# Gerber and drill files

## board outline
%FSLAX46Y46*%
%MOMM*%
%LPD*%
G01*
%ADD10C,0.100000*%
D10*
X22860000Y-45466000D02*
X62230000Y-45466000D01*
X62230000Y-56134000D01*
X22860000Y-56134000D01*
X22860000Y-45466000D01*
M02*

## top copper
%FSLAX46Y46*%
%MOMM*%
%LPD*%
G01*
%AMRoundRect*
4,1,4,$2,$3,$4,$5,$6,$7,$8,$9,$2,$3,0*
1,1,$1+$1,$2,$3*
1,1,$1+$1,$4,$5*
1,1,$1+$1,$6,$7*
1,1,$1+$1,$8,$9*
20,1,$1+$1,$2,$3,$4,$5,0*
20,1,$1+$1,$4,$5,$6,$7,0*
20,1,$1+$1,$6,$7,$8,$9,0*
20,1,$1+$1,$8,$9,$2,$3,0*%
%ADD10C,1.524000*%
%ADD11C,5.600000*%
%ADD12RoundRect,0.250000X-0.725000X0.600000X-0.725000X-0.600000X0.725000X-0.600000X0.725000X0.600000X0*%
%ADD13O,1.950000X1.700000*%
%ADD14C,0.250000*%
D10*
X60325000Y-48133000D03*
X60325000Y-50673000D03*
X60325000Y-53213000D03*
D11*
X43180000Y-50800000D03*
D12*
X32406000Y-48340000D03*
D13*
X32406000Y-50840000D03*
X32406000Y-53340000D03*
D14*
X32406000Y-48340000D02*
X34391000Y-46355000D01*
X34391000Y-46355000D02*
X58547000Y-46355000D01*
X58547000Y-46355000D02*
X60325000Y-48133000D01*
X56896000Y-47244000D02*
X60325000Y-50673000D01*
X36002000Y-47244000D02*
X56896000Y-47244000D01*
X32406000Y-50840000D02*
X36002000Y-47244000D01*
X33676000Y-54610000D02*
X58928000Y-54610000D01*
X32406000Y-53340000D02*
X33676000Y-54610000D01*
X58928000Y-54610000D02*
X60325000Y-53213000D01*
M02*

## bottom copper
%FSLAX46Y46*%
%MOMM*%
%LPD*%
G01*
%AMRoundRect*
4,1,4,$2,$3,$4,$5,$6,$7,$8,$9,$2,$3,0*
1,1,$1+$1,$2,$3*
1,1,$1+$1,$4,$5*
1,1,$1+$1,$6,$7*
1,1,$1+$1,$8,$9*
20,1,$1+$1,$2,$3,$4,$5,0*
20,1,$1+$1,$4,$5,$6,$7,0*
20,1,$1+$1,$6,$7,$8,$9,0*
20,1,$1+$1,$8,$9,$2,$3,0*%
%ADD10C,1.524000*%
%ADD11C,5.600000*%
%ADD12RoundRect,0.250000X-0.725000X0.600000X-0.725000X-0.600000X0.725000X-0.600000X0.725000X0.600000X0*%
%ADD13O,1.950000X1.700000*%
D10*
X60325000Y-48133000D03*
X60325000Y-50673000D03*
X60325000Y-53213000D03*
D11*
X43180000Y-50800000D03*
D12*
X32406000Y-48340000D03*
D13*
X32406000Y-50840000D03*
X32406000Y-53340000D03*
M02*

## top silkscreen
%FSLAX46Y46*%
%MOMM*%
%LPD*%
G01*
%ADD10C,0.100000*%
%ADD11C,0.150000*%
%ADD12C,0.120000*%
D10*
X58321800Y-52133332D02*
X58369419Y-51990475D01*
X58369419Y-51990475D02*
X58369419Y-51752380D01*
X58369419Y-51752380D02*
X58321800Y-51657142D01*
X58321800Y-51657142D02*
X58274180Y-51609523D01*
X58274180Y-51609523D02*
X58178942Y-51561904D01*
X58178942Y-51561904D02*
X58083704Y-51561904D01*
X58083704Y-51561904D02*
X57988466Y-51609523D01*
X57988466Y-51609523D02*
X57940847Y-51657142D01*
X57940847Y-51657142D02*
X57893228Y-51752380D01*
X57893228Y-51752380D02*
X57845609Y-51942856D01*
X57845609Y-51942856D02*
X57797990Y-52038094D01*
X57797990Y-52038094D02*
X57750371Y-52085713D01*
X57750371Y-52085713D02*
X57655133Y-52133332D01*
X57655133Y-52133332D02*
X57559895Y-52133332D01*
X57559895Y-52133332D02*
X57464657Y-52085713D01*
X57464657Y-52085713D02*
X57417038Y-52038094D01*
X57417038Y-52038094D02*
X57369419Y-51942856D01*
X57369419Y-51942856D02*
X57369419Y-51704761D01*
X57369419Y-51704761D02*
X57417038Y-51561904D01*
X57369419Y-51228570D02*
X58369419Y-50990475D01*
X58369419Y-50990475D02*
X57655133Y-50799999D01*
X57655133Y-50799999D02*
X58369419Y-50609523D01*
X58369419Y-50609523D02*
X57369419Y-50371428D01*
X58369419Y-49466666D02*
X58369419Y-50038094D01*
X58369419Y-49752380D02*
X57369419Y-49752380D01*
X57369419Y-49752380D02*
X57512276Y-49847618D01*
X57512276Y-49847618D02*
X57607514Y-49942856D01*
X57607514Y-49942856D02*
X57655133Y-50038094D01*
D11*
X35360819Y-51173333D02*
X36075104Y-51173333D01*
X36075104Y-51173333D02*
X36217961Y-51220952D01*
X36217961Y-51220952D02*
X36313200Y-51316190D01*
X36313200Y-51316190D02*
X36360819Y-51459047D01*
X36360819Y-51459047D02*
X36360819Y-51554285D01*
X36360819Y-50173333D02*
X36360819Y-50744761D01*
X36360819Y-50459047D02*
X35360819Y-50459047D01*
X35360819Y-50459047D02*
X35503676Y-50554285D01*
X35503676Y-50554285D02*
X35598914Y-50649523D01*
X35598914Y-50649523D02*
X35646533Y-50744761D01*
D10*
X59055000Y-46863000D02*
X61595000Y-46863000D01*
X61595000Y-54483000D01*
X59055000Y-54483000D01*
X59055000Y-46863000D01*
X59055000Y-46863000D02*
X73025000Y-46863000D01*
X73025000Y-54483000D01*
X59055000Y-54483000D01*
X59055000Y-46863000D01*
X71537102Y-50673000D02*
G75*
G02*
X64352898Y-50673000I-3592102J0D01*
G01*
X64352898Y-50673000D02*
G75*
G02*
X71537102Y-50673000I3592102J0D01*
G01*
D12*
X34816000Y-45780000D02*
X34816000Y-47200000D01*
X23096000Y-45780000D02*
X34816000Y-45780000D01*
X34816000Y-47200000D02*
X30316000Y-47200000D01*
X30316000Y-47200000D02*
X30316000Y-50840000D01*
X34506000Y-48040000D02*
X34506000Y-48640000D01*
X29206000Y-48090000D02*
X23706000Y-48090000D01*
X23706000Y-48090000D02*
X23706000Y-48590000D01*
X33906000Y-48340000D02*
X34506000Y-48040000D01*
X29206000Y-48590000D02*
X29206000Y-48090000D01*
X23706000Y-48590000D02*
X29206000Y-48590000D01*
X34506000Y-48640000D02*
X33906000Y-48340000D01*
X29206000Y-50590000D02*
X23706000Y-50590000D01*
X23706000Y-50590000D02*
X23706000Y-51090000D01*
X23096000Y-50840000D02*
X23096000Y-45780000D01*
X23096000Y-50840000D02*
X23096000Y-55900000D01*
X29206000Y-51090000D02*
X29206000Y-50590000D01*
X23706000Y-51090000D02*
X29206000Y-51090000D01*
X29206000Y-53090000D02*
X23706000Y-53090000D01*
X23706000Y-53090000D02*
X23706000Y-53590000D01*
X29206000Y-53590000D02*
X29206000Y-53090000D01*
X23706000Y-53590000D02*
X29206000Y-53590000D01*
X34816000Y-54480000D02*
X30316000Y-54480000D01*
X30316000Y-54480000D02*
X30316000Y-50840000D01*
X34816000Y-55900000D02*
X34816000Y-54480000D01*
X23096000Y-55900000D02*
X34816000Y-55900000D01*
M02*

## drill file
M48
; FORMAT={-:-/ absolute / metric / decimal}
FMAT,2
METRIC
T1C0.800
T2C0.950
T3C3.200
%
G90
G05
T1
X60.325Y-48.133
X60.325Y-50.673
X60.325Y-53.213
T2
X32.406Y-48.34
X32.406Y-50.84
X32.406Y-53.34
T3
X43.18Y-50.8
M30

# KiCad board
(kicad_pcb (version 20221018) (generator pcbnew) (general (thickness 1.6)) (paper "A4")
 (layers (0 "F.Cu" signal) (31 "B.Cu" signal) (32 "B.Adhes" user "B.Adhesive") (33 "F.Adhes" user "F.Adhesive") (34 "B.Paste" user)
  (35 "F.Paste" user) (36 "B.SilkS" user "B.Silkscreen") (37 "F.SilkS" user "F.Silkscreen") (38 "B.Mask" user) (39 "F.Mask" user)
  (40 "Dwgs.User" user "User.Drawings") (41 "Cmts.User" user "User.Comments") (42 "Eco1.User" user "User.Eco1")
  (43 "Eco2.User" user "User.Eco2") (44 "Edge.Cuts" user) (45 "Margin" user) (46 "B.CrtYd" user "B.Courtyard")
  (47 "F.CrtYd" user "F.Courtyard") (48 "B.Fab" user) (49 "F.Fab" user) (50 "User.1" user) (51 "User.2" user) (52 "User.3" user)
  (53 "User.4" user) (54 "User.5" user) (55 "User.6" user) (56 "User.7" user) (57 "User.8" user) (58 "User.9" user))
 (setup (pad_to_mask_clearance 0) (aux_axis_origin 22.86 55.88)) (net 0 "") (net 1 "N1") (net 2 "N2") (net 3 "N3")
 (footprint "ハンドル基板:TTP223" (layer "F.Cu") (at 60.325 46.863)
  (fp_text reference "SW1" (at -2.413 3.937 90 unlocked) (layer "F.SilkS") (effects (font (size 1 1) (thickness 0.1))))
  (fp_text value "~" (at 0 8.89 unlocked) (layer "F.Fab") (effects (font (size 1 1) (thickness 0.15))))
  (fp_rect (start -1.27 0) (end 1.27 7.62) (stroke (width 0.1) (type default)) (fill none) (layer "F.SilkS"))
  (fp_rect (start -1.27 0) (end 12.7 7.62) (stroke (width 0.1) (type default)) (fill none) (layer "F.SilkS"))
  (fp_circle (center 7.62 3.81) (end 10.16 6.35) (stroke (width 0.1) (type default)) (fill none) (layer "F.SilkS"))
  (pad "1" thru_hole circle (at 0 1.27) (size 1.524 1.524) (drill 0.8) (layers "*.Cu" "*.Mask") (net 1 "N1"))
  (pad "2" thru_hole circle (at 0 3.81) (size 1.524 1.524) (drill 0.8) (layers "*.Cu" "*.Mask") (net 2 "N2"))
  (pad "3" thru_hole circle (at 0 6.35) (size 1.524 1.524) (drill 0.8) (layers "*.Cu" "*.Mask") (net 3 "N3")))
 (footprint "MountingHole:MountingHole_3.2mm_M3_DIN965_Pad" (layer "F.Cu") (at 43.18 50.8)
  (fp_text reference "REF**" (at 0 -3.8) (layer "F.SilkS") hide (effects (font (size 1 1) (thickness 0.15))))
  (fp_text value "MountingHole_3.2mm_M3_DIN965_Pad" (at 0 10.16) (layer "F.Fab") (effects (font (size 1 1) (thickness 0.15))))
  (pad "1" thru_hole circle (at 0 0) (size 5.6 5.6) (drill 3.2) (layers "*.Cu" "*.Mask")))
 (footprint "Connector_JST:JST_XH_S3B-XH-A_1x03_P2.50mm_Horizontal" (layer "F.Cu") (at 32.406 48.34 -90)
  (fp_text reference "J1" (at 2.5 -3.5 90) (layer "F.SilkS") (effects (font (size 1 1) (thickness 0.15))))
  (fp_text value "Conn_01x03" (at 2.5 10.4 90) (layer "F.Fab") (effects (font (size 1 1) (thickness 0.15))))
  (fp_line (start -2.56 -2.41) (end -1.14 -2.41) (stroke (width 0.12) (type solid)) (layer "F.SilkS"))
  (fp_line (start -2.56 9.31) (end -2.56 -2.41) (stroke (width 0.12) (type solid)) (layer "F.SilkS"))
  (fp_line (start -1.14 -2.41) (end -1.14 2.09) (stroke (width 0.12) (type solid)) (layer "F.SilkS"))
  (fp_line (start -1.14 2.09) (end 2.5 2.09) (stroke (width 0.12) (type solid)) (layer "F.SilkS"))
  (fp_line (start -0.3 -2.1) (end 0.3 -2.1) (stroke (width 0.12) (type solid)) (layer "F.SilkS"))
  (fp_line (start -0.25 3.2) (end -0.25 8.7) (stroke (width 0.12) (type solid)) (layer "F.SilkS"))
  (fp_line (start -0.25 8.7) (end 0.25 8.7) (stroke (width 0.12) (type solid)) (layer "F.SilkS"))
  (fp_line (start 0 -1.5) (end -0.3 -2.1) (stroke (width 0.12) (type solid)) (layer "F.SilkS"))
  (fp_line (start 0.25 3.2) (end -0.25 3.2) (stroke (width 0.12) (type solid)) (layer "F.SilkS"))
  (fp_line (start 0.25 8.7) (end 0.25 3.2) (stroke (width 0.12) (type solid)) (layer "F.SilkS"))
  (fp_line (start 0.3 -2.1) (end 0 -1.5) (stroke (width 0.12) (type solid)) (layer "F.SilkS"))
  (fp_line (start 2.25 3.2) (end 2.25 8.7) (stroke (width 0.12) (type solid)) (layer "F.SilkS"))
  (fp_line (start 2.25 8.7) (end 2.75 8.7) (stroke (width 0.12) (type solid)) (layer "F.SilkS"))
  (fp_line (start 2.5 9.31) (end -2.56 9.31) (stroke (width 0.12) (type solid)) (layer "F.SilkS"))
  (fp_line (start 2.5 9.31) (end 7.56 9.31) (stroke (width 0.12) (type solid)) (layer "F.SilkS"))
  (fp_line (start 2.75 3.2) (end 2.25 3.2) (stroke (width 0.12) (type solid)) (layer "F.SilkS"))
  (fp_line (start 2.75 8.7) (end 2.75 3.2) (stroke (width 0.12) (type solid)) (layer "F.SilkS"))
  (fp_line (start 4.75 3.2) (end 4.75 8.7) (stroke (width 0.12) (type solid)) (layer "F.SilkS"))
  (fp_line (start 4.75 8.7) (end 5.25 8.7) (stroke (width 0.12) (type solid)) (layer "F.SilkS"))
  (fp_line (start 5.25 3.2) (end 4.75 3.2) (stroke (width 0.12) (type solid)) (layer "F.SilkS"))
  (fp_line (start 5.25 8.7) (end 5.25 3.2) (stroke (width 0.12) (type solid)) (layer "F.SilkS"))
  (fp_line (start 6.14 -2.41) (end 6.14 2.09) (stroke (width 0.12) (type solid)) (layer "F.SilkS"))
  (fp_line (start 6.14 2.09) (end 2.5 2.09) (stroke (width 0.12) (type solid)) (layer "F.SilkS"))
  (fp_line (start 7.56 -2.41) (end 6.14 -2.41) (stroke (width 0.12) (type solid)) (layer "F.SilkS"))
  (fp_line (start 7.56 9.31) (end 7.56 -2.41) (stroke (width 0.12) (type solid)) (layer "F.SilkS"))
  (pad "1" thru_hole roundrect (at 0 0 270) (size 1.7 1.95) (drill 0.95) (layers "*.Cu" "*.Mask") (roundrect_rratio 0.1470588235)
   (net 1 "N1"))
  (pad "2" thru_hole oval (at 2.5 0 270) (size 1.7 1.95) (drill 0.95) (layers "*.Cu" "*.Mask") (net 2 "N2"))
  (pad "3" thru_hole oval (at 5 0 270) (size 1.7 1.95) (drill 0.95) (layers "*.Cu" "*.Mask") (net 3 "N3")))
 (gr_rect (start 22.86 45.466) (end 62.23 56.134) (stroke (width 0.1) (type default)) (fill none) (layer "Edge.Cuts"))
 (segment (start 32.406 48.34) (end 34.391 46.355) (width 0.25) (layer "F.Cu") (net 1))
 (segment (start 34.391 46.355) (end 58.547 46.355) (width 0.25) (layer "F.Cu") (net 1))
 (segment (start 58.547 46.355) (end 60.325 48.133) (width 0.25) (layer "F.Cu") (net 1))
 (segment (start 56.896 47.244) (end 60.325 50.673) (width 0.25) (layer "F.Cu") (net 2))
 (segment (start 36.002 47.244) (end 56.896 47.244) (width 0.25) (layer "F.Cu") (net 2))
 (segment (start 32.406 50.84) (end 36.002 47.244) (width 0.25) (layer "F.Cu") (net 2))
 (segment (start 33.676 54.61) (end 58.928 54.61) (width 0.25) (layer "F.Cu") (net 3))
 (segment (start 32.406 53.34) (end 33.676 54.61) (width 0.25) (layer "F.Cu") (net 3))
 (segment (start 58.928 54.61) (end 60.325 53.213) (width 0.25) (layer "F.Cu") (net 3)))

